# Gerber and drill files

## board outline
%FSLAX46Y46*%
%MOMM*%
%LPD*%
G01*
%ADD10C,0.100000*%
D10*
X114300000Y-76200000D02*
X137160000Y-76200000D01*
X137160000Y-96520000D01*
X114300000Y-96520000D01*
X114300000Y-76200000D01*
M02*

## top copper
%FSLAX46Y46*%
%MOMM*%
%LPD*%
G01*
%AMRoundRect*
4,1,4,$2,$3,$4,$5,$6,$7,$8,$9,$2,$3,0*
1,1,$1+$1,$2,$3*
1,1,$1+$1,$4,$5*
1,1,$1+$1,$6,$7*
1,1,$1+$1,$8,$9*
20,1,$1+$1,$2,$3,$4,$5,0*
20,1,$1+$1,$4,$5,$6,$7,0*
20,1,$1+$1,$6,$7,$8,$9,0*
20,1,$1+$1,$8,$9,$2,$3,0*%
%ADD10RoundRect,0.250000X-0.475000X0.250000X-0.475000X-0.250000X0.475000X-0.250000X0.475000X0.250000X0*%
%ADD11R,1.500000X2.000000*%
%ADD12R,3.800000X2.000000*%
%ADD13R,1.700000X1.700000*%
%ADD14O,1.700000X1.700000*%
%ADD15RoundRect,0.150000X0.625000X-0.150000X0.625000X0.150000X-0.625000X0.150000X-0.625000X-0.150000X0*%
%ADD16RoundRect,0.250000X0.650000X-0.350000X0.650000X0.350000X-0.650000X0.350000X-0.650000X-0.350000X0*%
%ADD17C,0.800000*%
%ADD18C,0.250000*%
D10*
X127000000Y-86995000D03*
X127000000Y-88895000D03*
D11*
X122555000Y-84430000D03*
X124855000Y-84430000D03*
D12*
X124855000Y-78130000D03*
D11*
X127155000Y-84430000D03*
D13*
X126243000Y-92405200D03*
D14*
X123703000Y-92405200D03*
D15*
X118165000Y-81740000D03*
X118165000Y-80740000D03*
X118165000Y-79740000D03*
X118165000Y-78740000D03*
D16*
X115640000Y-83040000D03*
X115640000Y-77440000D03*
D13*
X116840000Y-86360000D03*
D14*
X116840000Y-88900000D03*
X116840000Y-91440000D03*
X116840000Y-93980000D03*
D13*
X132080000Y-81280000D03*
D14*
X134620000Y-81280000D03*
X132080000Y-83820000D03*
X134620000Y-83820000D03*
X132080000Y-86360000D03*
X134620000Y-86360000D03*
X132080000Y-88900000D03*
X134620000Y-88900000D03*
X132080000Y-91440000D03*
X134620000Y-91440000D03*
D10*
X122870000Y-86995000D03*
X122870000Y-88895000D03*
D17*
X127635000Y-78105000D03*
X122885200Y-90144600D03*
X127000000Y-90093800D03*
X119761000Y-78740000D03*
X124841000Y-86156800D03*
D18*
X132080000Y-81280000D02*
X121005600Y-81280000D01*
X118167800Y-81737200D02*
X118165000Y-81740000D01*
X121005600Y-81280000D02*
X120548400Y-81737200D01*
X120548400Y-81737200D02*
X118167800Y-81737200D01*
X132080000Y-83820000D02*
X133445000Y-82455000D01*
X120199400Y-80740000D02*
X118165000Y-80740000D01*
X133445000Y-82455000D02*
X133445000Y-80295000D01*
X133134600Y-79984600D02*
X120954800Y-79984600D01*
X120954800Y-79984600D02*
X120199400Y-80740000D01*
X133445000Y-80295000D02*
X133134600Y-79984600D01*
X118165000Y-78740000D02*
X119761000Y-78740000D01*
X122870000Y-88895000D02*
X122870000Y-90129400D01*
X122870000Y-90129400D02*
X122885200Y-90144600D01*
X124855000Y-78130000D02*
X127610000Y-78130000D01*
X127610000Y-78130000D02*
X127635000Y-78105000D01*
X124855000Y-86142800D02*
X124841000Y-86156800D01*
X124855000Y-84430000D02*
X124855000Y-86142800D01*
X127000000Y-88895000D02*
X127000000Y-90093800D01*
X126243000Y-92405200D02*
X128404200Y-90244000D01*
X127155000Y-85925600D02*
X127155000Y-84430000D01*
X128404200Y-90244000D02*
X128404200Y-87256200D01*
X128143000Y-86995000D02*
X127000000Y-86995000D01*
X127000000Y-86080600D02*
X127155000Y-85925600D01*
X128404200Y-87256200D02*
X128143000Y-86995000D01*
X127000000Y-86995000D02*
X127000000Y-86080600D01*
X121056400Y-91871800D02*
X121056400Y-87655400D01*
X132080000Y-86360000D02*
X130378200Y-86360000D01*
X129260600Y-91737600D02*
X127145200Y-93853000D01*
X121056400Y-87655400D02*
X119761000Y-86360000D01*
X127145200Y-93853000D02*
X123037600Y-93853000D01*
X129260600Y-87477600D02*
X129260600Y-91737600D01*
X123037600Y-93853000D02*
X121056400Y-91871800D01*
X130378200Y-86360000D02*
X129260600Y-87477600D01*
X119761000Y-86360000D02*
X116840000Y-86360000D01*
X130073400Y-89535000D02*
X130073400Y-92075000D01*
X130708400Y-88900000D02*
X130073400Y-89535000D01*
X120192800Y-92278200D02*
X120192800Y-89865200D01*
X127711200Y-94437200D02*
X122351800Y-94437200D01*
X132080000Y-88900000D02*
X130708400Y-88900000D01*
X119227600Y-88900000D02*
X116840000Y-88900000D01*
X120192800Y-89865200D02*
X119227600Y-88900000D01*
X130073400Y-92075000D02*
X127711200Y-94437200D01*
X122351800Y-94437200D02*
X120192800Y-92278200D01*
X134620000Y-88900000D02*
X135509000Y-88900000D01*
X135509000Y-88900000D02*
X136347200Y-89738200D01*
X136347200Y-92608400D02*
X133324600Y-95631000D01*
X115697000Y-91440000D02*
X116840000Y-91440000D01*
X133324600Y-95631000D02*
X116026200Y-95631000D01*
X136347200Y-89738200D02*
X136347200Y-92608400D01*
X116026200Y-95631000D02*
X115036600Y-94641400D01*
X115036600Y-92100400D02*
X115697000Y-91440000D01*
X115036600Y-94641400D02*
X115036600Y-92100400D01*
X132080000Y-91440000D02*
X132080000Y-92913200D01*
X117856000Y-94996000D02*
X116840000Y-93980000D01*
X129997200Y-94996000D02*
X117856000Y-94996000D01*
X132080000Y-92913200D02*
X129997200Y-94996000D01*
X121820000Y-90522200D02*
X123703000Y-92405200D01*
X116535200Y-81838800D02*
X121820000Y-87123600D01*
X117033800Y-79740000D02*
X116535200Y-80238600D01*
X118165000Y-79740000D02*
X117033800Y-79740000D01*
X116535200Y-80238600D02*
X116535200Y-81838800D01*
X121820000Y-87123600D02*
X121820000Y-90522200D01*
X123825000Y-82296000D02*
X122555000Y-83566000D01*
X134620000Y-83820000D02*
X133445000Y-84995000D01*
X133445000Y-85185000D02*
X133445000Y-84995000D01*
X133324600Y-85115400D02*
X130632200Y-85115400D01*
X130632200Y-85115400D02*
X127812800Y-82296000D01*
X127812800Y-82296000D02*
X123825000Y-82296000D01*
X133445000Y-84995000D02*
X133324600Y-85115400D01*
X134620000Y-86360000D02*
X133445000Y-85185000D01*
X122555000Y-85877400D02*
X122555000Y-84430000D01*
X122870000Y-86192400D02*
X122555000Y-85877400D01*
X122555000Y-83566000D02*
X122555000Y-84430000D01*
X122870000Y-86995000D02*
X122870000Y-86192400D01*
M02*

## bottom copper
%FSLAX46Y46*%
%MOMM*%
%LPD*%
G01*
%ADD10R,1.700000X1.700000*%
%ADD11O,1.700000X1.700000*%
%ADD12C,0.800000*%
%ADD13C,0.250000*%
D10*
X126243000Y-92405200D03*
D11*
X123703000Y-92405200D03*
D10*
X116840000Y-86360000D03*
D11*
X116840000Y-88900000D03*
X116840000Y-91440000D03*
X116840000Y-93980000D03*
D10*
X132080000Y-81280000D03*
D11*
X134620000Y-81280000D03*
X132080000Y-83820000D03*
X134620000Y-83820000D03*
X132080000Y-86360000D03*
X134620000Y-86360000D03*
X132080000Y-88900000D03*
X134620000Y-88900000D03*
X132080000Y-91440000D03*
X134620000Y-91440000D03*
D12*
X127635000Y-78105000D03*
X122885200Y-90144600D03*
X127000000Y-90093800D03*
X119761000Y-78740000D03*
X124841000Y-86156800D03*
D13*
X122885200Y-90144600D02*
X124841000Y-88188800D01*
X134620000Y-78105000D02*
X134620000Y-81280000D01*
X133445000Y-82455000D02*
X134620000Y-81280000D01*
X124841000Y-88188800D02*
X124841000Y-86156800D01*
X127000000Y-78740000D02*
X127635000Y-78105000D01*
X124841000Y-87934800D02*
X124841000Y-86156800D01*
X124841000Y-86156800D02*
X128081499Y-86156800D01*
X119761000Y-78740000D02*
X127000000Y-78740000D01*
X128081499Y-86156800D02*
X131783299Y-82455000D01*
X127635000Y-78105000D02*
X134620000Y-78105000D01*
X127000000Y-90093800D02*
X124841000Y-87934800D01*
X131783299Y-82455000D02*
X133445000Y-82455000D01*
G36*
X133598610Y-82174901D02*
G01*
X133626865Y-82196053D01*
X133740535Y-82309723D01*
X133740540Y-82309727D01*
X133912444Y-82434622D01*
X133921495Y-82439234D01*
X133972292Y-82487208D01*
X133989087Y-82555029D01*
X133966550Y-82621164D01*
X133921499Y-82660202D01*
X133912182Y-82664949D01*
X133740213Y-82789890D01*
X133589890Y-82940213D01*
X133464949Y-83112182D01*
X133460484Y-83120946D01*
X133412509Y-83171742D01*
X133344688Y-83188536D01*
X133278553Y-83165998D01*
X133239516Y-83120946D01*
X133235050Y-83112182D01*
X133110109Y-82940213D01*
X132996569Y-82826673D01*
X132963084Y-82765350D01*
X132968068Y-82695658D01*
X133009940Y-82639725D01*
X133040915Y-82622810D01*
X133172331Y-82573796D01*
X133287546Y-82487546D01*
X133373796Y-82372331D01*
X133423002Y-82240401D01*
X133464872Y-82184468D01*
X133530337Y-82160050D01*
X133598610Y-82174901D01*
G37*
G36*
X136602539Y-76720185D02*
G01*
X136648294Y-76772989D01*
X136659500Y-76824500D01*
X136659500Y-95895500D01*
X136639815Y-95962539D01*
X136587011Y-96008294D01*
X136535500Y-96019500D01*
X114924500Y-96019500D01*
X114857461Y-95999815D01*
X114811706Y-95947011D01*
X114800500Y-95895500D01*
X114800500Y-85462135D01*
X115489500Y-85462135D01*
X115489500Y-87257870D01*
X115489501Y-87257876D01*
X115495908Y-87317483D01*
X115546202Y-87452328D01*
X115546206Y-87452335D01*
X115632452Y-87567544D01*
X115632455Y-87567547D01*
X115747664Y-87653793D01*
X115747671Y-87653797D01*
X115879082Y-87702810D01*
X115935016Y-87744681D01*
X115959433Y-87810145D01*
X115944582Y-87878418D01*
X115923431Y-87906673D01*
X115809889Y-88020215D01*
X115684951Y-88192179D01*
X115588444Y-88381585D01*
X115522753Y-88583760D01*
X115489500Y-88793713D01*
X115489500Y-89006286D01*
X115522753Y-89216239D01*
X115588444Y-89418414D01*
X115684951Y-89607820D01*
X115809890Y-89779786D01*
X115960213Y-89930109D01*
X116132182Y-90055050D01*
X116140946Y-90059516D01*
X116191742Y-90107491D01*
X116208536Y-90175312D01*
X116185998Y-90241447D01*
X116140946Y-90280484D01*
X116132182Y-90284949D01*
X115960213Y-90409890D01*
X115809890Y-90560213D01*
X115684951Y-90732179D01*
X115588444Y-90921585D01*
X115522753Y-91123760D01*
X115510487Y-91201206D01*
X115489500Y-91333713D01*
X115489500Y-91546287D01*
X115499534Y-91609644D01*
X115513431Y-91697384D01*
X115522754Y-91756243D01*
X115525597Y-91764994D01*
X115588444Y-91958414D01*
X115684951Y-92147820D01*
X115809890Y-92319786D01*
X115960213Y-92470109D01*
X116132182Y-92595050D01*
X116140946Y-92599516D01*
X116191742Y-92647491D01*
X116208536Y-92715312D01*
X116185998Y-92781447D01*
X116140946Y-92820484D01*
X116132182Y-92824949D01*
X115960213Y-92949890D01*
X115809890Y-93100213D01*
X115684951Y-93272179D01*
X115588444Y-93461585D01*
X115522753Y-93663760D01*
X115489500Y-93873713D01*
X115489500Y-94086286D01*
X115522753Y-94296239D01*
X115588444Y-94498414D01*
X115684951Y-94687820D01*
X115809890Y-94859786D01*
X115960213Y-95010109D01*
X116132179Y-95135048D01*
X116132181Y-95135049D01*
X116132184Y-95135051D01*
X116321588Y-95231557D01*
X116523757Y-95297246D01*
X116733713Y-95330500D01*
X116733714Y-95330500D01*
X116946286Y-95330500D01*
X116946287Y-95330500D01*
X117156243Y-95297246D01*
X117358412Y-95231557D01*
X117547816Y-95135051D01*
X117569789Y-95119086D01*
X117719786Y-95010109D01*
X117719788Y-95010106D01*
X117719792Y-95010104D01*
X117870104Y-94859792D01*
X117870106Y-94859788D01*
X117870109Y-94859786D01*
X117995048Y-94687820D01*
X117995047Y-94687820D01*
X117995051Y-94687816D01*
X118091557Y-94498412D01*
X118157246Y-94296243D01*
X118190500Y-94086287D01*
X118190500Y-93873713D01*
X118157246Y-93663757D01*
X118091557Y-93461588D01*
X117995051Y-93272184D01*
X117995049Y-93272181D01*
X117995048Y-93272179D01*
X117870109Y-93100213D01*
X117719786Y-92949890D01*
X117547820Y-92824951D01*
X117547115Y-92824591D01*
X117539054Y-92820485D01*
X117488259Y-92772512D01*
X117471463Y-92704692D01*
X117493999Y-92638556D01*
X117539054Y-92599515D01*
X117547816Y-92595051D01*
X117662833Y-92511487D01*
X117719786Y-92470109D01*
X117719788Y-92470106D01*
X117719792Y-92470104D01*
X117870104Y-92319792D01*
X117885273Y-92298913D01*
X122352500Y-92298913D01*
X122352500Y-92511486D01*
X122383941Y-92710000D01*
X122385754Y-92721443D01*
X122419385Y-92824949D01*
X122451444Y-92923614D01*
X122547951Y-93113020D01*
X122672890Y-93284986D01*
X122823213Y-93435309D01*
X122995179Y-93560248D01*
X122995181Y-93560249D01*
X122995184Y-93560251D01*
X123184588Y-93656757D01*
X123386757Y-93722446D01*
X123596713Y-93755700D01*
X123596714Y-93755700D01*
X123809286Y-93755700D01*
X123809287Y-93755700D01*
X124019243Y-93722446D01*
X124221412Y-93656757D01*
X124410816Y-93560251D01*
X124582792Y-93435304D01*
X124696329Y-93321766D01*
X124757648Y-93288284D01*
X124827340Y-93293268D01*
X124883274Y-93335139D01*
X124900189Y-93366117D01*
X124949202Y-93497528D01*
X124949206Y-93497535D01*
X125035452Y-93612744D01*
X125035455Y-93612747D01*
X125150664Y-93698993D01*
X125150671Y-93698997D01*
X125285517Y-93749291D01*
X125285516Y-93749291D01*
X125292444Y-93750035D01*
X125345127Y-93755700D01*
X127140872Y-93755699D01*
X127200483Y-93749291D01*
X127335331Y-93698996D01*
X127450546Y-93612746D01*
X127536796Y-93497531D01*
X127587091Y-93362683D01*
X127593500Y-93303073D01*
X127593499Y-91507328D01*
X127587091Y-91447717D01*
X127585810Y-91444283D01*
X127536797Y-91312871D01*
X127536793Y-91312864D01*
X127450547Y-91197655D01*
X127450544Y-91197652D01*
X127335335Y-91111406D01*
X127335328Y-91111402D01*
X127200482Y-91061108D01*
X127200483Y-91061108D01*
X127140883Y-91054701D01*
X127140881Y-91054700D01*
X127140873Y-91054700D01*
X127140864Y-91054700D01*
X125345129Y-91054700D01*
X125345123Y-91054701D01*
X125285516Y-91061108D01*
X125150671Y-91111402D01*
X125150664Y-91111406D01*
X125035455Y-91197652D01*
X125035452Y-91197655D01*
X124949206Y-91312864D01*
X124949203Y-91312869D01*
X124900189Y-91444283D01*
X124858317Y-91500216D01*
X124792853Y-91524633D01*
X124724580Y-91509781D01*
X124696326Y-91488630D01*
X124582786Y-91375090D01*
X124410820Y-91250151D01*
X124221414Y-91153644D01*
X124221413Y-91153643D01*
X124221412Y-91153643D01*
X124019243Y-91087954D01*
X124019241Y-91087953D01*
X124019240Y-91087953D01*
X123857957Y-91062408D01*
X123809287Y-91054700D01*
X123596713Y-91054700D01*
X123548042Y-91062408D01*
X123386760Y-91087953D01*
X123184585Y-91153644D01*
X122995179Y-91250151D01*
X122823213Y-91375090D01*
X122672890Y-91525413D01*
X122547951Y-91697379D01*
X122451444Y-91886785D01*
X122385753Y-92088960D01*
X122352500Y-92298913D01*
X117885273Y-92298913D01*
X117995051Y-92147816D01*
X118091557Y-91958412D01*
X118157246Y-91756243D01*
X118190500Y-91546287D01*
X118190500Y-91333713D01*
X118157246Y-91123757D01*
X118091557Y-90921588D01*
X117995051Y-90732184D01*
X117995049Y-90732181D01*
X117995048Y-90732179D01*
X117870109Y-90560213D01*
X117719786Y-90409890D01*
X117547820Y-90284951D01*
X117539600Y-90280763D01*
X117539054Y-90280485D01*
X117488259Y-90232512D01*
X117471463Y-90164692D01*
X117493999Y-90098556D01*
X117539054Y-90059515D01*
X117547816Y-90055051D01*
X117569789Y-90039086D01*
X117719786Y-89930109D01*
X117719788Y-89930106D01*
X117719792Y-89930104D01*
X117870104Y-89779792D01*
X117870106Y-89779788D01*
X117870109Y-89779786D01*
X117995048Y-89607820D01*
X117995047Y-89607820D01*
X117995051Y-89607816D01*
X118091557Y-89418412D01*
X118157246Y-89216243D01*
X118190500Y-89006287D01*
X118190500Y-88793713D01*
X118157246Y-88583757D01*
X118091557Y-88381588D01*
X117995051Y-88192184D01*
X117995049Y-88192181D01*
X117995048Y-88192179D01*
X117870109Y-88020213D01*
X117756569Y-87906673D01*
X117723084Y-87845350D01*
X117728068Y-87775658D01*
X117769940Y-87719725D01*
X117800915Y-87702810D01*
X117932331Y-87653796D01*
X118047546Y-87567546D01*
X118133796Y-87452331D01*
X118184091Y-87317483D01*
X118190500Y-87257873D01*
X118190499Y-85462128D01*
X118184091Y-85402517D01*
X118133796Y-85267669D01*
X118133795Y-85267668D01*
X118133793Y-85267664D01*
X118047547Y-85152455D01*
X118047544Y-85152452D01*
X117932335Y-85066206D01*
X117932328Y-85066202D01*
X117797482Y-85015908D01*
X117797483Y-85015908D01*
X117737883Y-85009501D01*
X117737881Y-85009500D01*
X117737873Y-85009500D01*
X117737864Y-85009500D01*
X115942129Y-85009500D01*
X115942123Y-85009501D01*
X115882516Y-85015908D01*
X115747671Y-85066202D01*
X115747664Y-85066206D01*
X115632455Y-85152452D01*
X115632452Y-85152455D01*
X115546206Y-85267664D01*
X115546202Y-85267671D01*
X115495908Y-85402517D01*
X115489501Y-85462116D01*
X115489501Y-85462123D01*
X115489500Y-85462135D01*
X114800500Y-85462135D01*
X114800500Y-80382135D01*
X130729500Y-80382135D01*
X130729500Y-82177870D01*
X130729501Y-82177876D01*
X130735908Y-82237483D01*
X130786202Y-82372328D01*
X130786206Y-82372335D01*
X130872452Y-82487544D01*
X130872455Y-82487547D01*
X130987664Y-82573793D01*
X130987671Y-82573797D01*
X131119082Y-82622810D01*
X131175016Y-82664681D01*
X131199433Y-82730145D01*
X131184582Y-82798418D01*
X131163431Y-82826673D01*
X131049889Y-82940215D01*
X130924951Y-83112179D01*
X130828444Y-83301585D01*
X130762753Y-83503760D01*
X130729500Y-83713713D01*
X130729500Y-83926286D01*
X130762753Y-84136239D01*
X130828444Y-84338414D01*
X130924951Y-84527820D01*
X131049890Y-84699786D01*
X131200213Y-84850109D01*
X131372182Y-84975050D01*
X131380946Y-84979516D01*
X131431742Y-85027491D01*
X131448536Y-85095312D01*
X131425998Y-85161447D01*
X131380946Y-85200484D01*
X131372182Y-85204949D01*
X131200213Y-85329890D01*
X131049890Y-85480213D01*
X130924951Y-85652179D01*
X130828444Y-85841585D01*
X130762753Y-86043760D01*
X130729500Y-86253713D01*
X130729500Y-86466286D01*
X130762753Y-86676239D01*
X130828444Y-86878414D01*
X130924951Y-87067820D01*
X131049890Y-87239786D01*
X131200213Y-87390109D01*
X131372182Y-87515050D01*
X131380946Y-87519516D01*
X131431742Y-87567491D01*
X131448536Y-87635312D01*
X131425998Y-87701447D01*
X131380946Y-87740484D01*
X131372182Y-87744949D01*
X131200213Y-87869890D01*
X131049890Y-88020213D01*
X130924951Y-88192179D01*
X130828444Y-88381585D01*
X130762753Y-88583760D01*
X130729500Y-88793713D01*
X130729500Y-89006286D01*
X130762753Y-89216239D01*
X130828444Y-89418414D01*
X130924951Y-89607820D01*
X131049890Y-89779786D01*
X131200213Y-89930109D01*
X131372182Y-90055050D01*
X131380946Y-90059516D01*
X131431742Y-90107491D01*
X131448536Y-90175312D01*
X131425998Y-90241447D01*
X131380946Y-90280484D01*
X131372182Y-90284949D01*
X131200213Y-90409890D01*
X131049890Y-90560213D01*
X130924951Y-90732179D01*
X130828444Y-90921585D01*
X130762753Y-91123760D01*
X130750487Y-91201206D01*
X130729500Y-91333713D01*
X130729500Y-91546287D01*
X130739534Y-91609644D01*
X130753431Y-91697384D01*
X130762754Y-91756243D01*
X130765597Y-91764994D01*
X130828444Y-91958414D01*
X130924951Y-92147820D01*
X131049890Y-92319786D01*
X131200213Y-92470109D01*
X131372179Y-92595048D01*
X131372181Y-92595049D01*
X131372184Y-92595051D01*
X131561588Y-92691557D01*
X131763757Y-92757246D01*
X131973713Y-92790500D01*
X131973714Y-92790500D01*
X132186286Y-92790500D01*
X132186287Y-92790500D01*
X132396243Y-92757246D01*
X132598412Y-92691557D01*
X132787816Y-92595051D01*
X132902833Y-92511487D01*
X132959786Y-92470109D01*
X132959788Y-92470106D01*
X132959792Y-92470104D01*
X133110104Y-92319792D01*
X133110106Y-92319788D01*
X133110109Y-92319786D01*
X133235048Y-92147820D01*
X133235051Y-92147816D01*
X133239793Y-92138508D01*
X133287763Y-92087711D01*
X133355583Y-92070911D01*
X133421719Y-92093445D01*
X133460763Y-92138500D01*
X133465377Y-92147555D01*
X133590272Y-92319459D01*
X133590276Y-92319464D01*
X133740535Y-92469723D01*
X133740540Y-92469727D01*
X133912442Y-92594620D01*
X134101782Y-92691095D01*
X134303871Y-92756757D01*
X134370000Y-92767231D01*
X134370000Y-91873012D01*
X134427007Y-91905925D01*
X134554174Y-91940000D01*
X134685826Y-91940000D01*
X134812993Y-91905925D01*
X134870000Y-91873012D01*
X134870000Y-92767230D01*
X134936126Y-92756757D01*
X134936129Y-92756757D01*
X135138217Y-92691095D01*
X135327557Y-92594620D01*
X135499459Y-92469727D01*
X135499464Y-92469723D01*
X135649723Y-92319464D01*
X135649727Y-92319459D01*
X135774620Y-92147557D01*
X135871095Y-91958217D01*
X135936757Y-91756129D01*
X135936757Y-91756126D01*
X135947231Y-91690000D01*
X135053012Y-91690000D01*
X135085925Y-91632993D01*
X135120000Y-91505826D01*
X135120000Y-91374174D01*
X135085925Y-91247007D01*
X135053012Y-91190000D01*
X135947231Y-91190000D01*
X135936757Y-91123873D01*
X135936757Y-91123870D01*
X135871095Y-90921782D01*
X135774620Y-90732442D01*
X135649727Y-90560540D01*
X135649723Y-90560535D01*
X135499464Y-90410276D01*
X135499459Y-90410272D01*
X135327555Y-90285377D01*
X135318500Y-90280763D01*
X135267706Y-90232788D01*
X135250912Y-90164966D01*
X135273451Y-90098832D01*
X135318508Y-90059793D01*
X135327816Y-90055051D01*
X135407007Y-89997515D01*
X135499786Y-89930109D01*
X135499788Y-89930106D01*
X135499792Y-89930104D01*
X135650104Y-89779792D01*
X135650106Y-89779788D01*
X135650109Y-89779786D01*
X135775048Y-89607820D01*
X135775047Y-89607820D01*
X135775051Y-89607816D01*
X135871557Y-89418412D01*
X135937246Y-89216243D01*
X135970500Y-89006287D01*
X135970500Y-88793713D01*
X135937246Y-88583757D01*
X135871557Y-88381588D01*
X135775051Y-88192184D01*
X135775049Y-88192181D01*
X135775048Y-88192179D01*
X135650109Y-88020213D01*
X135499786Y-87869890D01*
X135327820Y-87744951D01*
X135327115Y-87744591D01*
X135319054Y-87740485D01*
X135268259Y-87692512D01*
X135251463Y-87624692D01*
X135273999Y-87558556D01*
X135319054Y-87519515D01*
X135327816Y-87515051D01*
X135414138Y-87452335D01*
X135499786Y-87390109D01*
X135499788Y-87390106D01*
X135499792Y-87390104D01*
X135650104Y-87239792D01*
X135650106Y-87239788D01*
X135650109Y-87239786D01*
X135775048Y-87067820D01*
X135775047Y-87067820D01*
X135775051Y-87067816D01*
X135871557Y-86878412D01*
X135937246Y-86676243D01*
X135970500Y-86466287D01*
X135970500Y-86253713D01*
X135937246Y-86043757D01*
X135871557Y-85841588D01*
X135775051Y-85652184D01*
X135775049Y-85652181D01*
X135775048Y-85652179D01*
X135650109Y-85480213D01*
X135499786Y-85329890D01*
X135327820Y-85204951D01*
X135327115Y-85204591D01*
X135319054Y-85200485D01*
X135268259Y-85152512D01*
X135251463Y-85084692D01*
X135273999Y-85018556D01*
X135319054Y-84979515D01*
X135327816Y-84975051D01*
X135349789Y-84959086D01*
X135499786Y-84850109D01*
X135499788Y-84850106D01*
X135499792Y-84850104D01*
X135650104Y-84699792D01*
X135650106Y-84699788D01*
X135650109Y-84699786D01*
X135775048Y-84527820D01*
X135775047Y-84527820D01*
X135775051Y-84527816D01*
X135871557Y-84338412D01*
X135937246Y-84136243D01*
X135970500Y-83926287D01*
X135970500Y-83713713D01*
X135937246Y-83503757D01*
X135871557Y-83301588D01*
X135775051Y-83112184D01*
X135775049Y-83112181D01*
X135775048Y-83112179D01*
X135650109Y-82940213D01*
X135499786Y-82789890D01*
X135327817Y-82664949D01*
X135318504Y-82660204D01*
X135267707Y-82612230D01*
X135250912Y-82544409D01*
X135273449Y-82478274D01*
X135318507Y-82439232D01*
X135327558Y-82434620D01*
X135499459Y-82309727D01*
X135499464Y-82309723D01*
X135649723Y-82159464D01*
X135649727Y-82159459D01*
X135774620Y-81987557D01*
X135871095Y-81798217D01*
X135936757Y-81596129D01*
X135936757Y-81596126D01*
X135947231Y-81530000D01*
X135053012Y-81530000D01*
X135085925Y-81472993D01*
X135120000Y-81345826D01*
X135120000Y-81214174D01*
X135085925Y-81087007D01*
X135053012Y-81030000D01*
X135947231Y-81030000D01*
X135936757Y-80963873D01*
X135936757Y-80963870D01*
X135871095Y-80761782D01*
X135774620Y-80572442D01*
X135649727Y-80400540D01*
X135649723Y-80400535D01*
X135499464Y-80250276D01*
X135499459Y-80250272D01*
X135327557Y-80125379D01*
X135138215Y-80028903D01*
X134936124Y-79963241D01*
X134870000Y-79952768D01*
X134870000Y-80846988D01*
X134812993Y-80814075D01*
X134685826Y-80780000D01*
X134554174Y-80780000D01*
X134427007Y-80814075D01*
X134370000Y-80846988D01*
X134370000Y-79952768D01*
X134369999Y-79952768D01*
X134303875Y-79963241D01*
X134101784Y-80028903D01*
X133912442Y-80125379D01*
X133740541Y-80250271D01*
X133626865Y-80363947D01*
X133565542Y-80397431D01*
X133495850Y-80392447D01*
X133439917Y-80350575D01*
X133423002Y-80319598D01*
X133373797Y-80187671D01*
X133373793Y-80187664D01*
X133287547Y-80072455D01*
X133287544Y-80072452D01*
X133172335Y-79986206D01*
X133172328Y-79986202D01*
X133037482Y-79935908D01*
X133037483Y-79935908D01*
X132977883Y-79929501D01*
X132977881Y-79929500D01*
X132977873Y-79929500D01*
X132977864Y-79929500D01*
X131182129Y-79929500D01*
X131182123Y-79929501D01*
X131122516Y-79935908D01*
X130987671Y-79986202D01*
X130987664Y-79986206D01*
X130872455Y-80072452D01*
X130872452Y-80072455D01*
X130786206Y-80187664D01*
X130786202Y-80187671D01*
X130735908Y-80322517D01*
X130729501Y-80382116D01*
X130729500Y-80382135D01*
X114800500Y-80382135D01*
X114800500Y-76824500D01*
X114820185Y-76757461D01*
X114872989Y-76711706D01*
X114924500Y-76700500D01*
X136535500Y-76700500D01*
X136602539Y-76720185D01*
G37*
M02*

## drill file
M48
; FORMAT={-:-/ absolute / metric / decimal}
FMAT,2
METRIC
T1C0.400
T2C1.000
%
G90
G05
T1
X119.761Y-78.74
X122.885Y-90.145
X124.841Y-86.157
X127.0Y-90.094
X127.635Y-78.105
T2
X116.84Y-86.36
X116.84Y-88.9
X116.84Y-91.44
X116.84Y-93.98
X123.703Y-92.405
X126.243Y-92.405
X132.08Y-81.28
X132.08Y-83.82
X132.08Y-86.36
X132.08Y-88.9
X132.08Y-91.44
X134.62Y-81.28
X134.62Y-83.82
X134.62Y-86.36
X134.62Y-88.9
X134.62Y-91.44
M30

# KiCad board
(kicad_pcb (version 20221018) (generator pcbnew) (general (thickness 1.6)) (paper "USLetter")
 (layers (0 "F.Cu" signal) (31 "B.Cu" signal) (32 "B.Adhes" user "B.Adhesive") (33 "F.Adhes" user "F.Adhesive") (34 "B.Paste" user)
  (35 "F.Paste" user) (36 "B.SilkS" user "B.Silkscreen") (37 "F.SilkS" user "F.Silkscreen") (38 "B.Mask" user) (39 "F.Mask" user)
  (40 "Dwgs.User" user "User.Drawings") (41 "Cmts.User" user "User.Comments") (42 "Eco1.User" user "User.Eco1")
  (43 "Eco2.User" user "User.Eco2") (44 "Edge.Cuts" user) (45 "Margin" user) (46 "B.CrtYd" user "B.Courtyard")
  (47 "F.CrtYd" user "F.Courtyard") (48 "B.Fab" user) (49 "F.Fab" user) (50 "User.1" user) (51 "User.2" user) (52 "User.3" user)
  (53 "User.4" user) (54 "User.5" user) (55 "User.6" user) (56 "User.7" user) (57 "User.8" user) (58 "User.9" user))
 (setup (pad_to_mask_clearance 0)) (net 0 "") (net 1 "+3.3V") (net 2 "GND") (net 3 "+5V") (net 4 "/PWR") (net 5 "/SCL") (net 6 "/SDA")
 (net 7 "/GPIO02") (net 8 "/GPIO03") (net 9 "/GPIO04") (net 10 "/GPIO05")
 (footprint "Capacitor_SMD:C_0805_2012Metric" (layer "F.Cu") (at 127 87.945 -90)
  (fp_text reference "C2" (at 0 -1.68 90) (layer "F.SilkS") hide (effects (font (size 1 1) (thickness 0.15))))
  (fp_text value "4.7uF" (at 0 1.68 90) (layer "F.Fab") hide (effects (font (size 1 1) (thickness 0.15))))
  (pad "1" smd roundrect (at -0.95 0 270) (size 1 1.45) (layers "F.Cu" "F.Paste" "F.Mask") (roundrect_rratio 0.25) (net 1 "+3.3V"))
  (pad "2" smd roundrect (at 0.95 0 270) (size 1 1.45) (layers "F.Cu" "F.Paste" "F.Mask") (roundrect_rratio 0.25) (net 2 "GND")))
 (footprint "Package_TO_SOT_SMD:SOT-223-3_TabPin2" (layer "F.Cu") (at 124.855 81.28 90)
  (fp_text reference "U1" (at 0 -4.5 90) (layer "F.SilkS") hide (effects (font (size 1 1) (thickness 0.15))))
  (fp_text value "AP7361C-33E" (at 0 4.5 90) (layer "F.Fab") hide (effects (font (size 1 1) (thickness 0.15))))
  (pad "1" smd rect (at -3.15 -2.3 90) (size 2 1.5) (layers "F.Cu" "F.Paste" "F.Mask") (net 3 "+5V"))
  (pad "2" smd rect (at -3.15 0 90) (size 2 1.5) (layers "F.Cu" "F.Paste" "F.Mask") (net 2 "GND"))
  (pad "2" smd rect (at 3.15 0 90) (size 2 3.8) (layers "F.Cu" "F.Paste" "F.Mask") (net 2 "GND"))
  (pad "3" smd rect (at -3.15 2.3 90) (size 2 1.5) (layers "F.Cu" "F.Paste" "F.Mask") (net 1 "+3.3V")))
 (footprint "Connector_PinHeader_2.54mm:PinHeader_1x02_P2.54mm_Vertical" (layer "F.Cu") (at 126.243 92.4052 -90)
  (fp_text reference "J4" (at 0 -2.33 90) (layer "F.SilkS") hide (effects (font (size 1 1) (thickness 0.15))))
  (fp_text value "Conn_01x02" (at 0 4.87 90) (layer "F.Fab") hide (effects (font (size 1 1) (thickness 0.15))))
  (pad "1" thru_hole rect (at 0 0 270) (size 1.7 1.7) (drill 1) (layers "*.Cu" "*.Mask") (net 1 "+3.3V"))
  (pad "2" thru_hole oval (at 0 2.54 270) (size 1.7 1.7) (drill 1) (layers "*.Cu" "*.Mask") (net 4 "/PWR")))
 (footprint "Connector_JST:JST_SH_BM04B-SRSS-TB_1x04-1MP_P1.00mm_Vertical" (layer "F.Cu") (at 116.84 80.24 90)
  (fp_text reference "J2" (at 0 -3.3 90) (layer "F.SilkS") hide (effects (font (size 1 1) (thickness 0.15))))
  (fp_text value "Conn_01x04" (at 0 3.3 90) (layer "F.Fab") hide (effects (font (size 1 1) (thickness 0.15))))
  (pad "1" smd roundrect (at -1.5 1.325 90) (size 0.6 1.55) (layers "F.Cu" "F.Paste" "F.Mask") (roundrect_rratio 0.25) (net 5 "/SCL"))
  (pad "2" smd roundrect (at -0.5 1.325 90) (size 0.6 1.55) (layers "F.Cu" "F.Paste" "F.Mask") (roundrect_rratio 0.25) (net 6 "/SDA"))
  (pad "3" smd roundrect (at 0.5 1.325 90) (size 0.6 1.55) (layers "F.Cu" "F.Paste" "F.Mask") (roundrect_rratio 0.25) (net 4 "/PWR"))
  (pad "4" smd roundrect (at 1.5 1.325 90) (size 0.6 1.55) (layers "F.Cu" "F.Paste" "F.Mask") (roundrect_rratio 0.25) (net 2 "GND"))
  (pad "MP" smd roundrect (at -2.8 -1.2 90) (size 1.2 1.8) (layers "F.Cu" "F.Paste" "F.Mask") (roundrect_rratio 0.208333))
  (pad "MP" smd roundrect (at 2.8 -1.2 90) (size 1.2 1.8) (layers "F.Cu" "F.Paste" "F.Mask") (roundrect_rratio 0.208333)))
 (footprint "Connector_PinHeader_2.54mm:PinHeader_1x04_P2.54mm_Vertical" (layer "F.Cu") (at 116.84 86.36)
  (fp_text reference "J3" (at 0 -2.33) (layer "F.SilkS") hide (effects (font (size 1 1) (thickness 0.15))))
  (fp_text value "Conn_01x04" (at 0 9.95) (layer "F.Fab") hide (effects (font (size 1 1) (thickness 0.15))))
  (pad "1" thru_hole rect (at 0 0) (size 1.7 1.7) (drill 1) (layers "*.Cu" "*.Mask") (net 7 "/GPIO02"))
  (pad "2" thru_hole oval (at 0 2.54) (size 1.7 1.7) (drill 1) (layers "*.Cu" "*.Mask") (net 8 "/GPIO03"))
  (pad "3" thru_hole oval (at 0 5.08) (size 1.7 1.7) (drill 1) (layers "*.Cu" "*.Mask") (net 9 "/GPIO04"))
  (pad "4" thru_hole oval (at 0 7.62) (size 1.7 1.7) (drill 1) (layers "*.Cu" "*.Mask") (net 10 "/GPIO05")))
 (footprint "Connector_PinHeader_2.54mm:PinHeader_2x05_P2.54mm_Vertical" (layer "F.Cu") (at 132.08 81.28)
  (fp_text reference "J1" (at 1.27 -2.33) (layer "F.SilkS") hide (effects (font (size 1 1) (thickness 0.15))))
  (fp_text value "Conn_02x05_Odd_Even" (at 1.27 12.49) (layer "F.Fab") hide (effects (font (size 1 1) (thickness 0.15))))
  (pad "1" thru_hole rect (at 0 0) (size 1.7 1.7) (drill 1) (layers "*.Cu" "*.Mask") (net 5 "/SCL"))
  (pad "2" thru_hole oval (at 2.54 0) (size 1.7 1.7) (drill 1) (layers "*.Cu" "*.Mask") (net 2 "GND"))
  (pad "3" thru_hole oval (at 0 2.54) (size 1.7 1.7) (drill 1) (layers "*.Cu" "*.Mask") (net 6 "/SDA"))
  (pad "4" thru_hole oval (at 2.54 2.54) (size 1.7 1.7) (drill 1) (layers "*.Cu" "*.Mask") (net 3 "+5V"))
  (pad "5" thru_hole oval (at 0 5.08) (size 1.7 1.7) (drill 1) (layers "*.Cu" "*.Mask") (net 7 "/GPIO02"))
  (pad "6" thru_hole oval (at 2.54 5.08) (size 1.7 1.7) (drill 1) (layers "*.Cu" "*.Mask") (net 3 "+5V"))
  (pad "7" thru_hole oval (at 0 7.62) (size 1.7 1.7) (drill 1) (layers "*.Cu" "*.Mask") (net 8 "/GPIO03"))
  (pad "8" thru_hole oval (at 2.54 7.62) (size 1.7 1.7) (drill 1) (layers "*.Cu" "*.Mask") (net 9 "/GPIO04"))
  (pad "9" thru_hole oval (at 0 10.16) (size 1.7 1.7) (drill 1) (layers "*.Cu" "*.Mask") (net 10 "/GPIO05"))
  (pad "10" thru_hole oval (at 2.54 10.16) (size 1.7 1.7) (drill 1) (layers "*.Cu" "*.Mask") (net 2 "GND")))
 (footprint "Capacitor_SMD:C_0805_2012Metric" (layer "F.Cu") (at 122.87 87.945 -90)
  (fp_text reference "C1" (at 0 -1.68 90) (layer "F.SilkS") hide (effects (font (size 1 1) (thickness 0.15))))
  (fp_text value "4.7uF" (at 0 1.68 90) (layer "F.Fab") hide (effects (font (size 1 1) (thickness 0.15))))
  (pad "1" smd roundrect (at -0.95 0 270) (size 1 1.45) (layers "F.Cu" "F.Paste" "F.Mask") (roundrect_rratio 0.25) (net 3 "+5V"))
  (pad "2" smd roundrect (at 0.95 0 270) (size 1 1.45) (layers "F.Cu" "F.Paste" "F.Mask") (roundrect_rratio 0.25) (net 2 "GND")))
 (gr_rect (start 114.3 76.2) (end 137.16 96.52) (stroke (width 0.1) (type default)) (fill none) (layer "Edge.Cuts"))
 (segment (start 132.08 81.28) (end 121.0056 81.28) (width 0.25) (layer "F.Cu") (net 5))
 (segment (start 118.1678 81.7372) (end 118.165 81.74) (width 0.25) (layer "F.Cu") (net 5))
 (segment (start 121.0056 81.28) (end 120.5484 81.7372) (width 0.25) (layer "F.Cu") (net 5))
 (segment (start 120.5484 81.7372) (end 118.1678 81.7372) (width 0.25) (layer "F.Cu") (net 5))
 (segment (start 132.08 83.82) (end 133.445 82.455) (width 0.25) (layer "F.Cu") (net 6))
 (segment (start 120.1994 80.74) (end 118.165 80.74) (width 0.25) (layer "F.Cu") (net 6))
 (segment (start 133.445 82.455) (end 133.445 80.295) (width 0.25) (layer "F.Cu") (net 6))
 (segment (start 133.1346 79.9846) (end 120.9548 79.9846) (width 0.25) (layer "F.Cu") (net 6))
 (segment (start 120.9548 79.9846) (end 120.1994 80.74) (width 0.25) (layer "F.Cu") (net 6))
 (segment (start 133.445 80.295) (end 133.1346 79.9846) (width 0.25) (layer "F.Cu") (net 6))
 (segment (start 118.165 78.74) (end 119.761 78.74) (width 0.25) (layer "F.Cu") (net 2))
 (segment (start 122.87 88.895) (end 122.87 90.1294) (width 0.25) (layer "F.Cu") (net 2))
 (segment (start 122.87 90.1294) (end 122.8852 90.1446) (width 0.25) (layer "F.Cu") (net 2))
 (segment (start 124.855 78.13) (end 127.61 78.13) (width 0.25) (layer "F.Cu") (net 2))
 (segment (start 127.61 78.13) (end 127.635 78.105) (width 0.25) (layer "F.Cu") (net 2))
 (segment (start 124.855 86.1428) (end 124.841 86.1568) (width 0.25) (layer "F.Cu") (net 2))
 (segment (start 124.855 84.43) (end 124.855 86.1428) (width 0.25) (layer "F.Cu") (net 2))
 (segment (start 127 88.895) (end 127 90.0938) (width 0.25) (layer "F.Cu") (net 2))
 (via (at 127.635 78.105) (size 0.8) (drill 0.4) (layers "F.Cu" "B.Cu") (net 2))
 (via (at 122.8852 90.1446) (size 0.8) (drill 0.4) (layers "F.Cu" "B.Cu") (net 2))
 (via (at 127 90.0938) (size 0.8) (drill 0.4) (layers "F.Cu" "B.Cu") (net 2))
 (via (at 119.761 78.74) (size 0.8) (drill 0.4) (layers "F.Cu" "B.Cu") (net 2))
 (via (at 124.841 86.1568) (size 0.8) (drill 0.4) (layers "F.Cu" "B.Cu") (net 2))
 (segment (start 122.8852 90.1446) (end 124.841 88.1888) (width 0.25) (layer "B.Cu") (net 2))
 (segment (start 134.62 78.105) (end 134.62 81.28) (width 0.25) (layer "B.Cu") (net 2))
 (segment (start 133.445 82.455) (end 134.62 81.28) (width 0.25) (layer "B.Cu") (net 2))
 (segment (start 124.841 88.1888) (end 124.841 86.1568) (width 0.25) (layer "B.Cu") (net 2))
 (segment (start 127 78.74) (end 127.635 78.105) (width 0.25) (layer "B.Cu") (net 2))
 (segment (start 124.841 87.9348) (end 124.841 86.1568) (width 0.25) (layer "B.Cu") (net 2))
 (segment (start 124.841 86.1568) (end 128.081499 86.1568) (width 0.25) (layer "B.Cu") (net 2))
 (segment (start 119.761 78.74) (end 127 78.74) (width 0.25) (layer "B.Cu") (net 2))
 (segment (start 128.081499 86.1568) (end 131.783299 82.455) (width 0.25) (layer "B.Cu") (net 2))
 (segment (start 127.635 78.105) (end 134.62 78.105) (width 0.25) (layer "B.Cu") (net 2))
 (segment (start 127 90.0938) (end 124.841 87.9348) (width 0.25) (layer "B.Cu") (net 2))
 (segment (start 131.783299 82.455) (end 133.445 82.455) (width 0.25) (layer "B.Cu") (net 2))
 (segment (start 126.243 92.4052) (end 128.4042 90.244) (width 0.25) (layer "F.Cu") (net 1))
 (segment (start 127.155 85.9256) (end 127.155 84.43) (width 0.25) (layer "F.Cu") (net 1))
 (segment (start 128.4042 90.244) (end 128.4042 87.2562) (width 0.25) (layer "F.Cu") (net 1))
 (segment (start 128.143 86.995) (end 127 86.995) (width 0.25) (layer "F.Cu") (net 1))
 (segment (start 127 86.0806) (end 127.155 85.9256) (width 0.25) (layer "F.Cu") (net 1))
 (segment (start 128.4042 87.2562) (end 128.143 86.995) (width 0.25) (layer "F.Cu") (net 1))
 (segment (start 127 86.995) (end 127 86.0806) (width 0.25) (layer "F.Cu") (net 1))
 (segment (start 121.0564 91.8718) (end 121.0564 87.6554) (width 0.25) (layer "F.Cu") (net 7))
 (segment (start 132.08 86.36) (end 130.3782 86.36) (width 0.25) (layer "F.Cu") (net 7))
 (segment (start 129.2606 91.7376) (end 127.1452 93.853) (width 0.25) (layer "F.Cu") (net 7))
 (segment (start 121.0564 87.6554) (end 119.761 86.36) (width 0.25) (layer "F.Cu") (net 7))
 (segment (start 127.1452 93.853) (end 123.0376 93.853) (width 0.25) (layer "F.Cu") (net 7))
 (segment (start 129.2606 87.4776) (end 129.2606 91.7376) (width 0.25) (layer "F.Cu") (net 7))
 (segment (start 123.0376 93.853) (end 121.0564 91.8718) (width 0.25) (layer "F.Cu") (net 7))
 (segment (start 130.3782 86.36) (end 129.2606 87.4776) (width 0.25) (layer "F.Cu") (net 7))
 (segment (start 119.761 86.36) (end 116.84 86.36) (width 0.25) (layer "F.Cu") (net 7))
 (segment (start 130.0734 89.535) (end 130.0734 92.075) (width 0.25) (layer "F.Cu") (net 8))
 (segment (start 130.7084 88.9) (end 130.0734 89.535) (width 0.25) (layer "F.Cu") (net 8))
 (segment (start 120.1928 92.2782) (end 120.1928 89.8652) (width 0.25) (layer "F.Cu") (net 8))
 (segment (start 127.7112 94.4372) (end 122.3518 94.4372) (width 0.25) (layer "F.Cu") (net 8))
 (segment (start 132.08 88.9) (end 130.7084 88.9) (width 0.25) (layer "F.Cu") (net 8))
 (segment (start 119.2276 88.9) (end 116.84 88.9) (width 0.25) (layer "F.Cu") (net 8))
 (segment (start 120.1928 89.8652) (end 119.2276 88.9) (width 0.25) (layer "F.Cu") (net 8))
 (segment (start 130.0734 92.075) (end 127.7112 94.4372) (width 0.25) (layer "F.Cu") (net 8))
 (segment (start 122.3518 94.4372) (end 120.1928 92.2782) (width 0.25) (layer "F.Cu") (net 8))
 (segment (start 134.62 88.9) (end 135.509 88.9) (width 0.25) (layer "F.Cu") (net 9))
 (segment (start 135.509 88.9) (end 136.3472 89.7382) (width 0.25) (layer "F.Cu") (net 9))
 (segment (start 136.3472 92.6084) (end 133.3246 95.631) (width 0.25) (layer "F.Cu") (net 9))
 (segment (start 115.697 91.44) (end 116.84 91.44) (width 0.25) (layer "F.Cu") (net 9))
 (segment (start 133.3246 95.631) (end 116.0262 95.631) (width 0.25) (layer "F.Cu") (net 9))
 (segment (start 136.3472 89.7382) (end 136.3472 92.6084) (width 0.25) (layer "F.Cu") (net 9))
 (segment (start 116.0262 95.631) (end 115.0366 94.6414) (width 0.25) (layer "F.Cu") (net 9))
 (segment (start 115.0366 92.1004) (end 115.697 91.44) (width 0.25) (layer "F.Cu") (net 9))
 (segment (start 115.0366 94.6414) (end 115.0366 92.1004) (width 0.25) (layer "F.Cu") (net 9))
 (segment (start 132.08 91.44) (end 132.08 92.9132) (width 0.25) (layer "F.Cu") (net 10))
 (segment (start 117.856 94.996) (end 116.84 93.98) (width 0.25) (layer "F.Cu") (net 10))
 (segment (start 129.9972 94.996) (end 117.856 94.996) (width 0.25) (layer "F.Cu") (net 10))
 (segment (start 132.08 92.9132) (end 129.9972 94.996) (width 0.25) (layer "F.Cu") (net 10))
 (segment (start 121.82 90.5222) (end 123.703 92.4052) (width 0.25) (layer "F.Cu") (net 4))
 (segment (start 116.5352 81.8388) (end 121.82 87.1236) (width 0.25) (layer "F.Cu") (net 4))
 (segment (start 117.0338 79.74) (end 116.5352 80.2386) (width 0.25) (layer "F.Cu") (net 4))
 (segment (start 118.165 79.74) (end 117.0338 79.74) (width 0.25) (layer "F.Cu") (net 4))
 (segment (start 116.5352 80.2386) (end 116.5352 81.8388) (width 0.25) (layer "F.Cu") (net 4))
 (segment (start 121.82 87.1236) (end 121.82 90.5222) (width 0.25) (layer "F.Cu") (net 4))
 (segment (start 123.825 82.296) (end 122.555 83.566) (width 0.25) (layer "F.Cu") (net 3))
 (segment (start 134.62 83.82) (end 133.445 84.995) (width 0.25) (layer "F.Cu") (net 3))
 (segment (start 133.445 85.185) (end 133.445 84.995) (width 0.25) (layer "F.Cu") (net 3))
 (segment (start 133.3246 85.1154) (end 130.6322 85.1154) (width 0.25) (layer "F.Cu") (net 3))
 (segment (start 130.6322 85.1154) (end 127.8128 82.296) (width 0.25) (layer "F.Cu") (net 3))
 (segment (start 127.8128 82.296) (end 123.825 82.296) (width 0.25) (layer "F.Cu") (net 3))
 (segment (start 133.445 84.995) (end 133.3246 85.1154) (width 0.25) (layer "F.Cu") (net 3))
 (segment (start 134.62 86.36) (end 133.445 85.185) (width 0.25) (layer "F.Cu") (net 3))
 (segment (start 122.555 85.8774) (end 122.555 84.43) (width 0.25) (layer "F.Cu") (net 3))
 (segment (start 122.87 86.1924) (end 122.555 85.8774) (width 0.25) (layer "F.Cu") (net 3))
 (segment (start 122.555 83.566) (end 122.555 84.43) (width 0.25) (layer "F.Cu") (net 3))
 (segment (start 122.87 86.995) (end 122.87 86.1924) (width 0.25) (layer "F.Cu") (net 3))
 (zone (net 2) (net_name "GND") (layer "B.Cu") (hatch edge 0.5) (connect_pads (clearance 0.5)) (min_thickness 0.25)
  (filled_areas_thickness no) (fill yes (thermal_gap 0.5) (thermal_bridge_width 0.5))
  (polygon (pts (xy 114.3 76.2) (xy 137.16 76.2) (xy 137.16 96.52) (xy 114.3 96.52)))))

